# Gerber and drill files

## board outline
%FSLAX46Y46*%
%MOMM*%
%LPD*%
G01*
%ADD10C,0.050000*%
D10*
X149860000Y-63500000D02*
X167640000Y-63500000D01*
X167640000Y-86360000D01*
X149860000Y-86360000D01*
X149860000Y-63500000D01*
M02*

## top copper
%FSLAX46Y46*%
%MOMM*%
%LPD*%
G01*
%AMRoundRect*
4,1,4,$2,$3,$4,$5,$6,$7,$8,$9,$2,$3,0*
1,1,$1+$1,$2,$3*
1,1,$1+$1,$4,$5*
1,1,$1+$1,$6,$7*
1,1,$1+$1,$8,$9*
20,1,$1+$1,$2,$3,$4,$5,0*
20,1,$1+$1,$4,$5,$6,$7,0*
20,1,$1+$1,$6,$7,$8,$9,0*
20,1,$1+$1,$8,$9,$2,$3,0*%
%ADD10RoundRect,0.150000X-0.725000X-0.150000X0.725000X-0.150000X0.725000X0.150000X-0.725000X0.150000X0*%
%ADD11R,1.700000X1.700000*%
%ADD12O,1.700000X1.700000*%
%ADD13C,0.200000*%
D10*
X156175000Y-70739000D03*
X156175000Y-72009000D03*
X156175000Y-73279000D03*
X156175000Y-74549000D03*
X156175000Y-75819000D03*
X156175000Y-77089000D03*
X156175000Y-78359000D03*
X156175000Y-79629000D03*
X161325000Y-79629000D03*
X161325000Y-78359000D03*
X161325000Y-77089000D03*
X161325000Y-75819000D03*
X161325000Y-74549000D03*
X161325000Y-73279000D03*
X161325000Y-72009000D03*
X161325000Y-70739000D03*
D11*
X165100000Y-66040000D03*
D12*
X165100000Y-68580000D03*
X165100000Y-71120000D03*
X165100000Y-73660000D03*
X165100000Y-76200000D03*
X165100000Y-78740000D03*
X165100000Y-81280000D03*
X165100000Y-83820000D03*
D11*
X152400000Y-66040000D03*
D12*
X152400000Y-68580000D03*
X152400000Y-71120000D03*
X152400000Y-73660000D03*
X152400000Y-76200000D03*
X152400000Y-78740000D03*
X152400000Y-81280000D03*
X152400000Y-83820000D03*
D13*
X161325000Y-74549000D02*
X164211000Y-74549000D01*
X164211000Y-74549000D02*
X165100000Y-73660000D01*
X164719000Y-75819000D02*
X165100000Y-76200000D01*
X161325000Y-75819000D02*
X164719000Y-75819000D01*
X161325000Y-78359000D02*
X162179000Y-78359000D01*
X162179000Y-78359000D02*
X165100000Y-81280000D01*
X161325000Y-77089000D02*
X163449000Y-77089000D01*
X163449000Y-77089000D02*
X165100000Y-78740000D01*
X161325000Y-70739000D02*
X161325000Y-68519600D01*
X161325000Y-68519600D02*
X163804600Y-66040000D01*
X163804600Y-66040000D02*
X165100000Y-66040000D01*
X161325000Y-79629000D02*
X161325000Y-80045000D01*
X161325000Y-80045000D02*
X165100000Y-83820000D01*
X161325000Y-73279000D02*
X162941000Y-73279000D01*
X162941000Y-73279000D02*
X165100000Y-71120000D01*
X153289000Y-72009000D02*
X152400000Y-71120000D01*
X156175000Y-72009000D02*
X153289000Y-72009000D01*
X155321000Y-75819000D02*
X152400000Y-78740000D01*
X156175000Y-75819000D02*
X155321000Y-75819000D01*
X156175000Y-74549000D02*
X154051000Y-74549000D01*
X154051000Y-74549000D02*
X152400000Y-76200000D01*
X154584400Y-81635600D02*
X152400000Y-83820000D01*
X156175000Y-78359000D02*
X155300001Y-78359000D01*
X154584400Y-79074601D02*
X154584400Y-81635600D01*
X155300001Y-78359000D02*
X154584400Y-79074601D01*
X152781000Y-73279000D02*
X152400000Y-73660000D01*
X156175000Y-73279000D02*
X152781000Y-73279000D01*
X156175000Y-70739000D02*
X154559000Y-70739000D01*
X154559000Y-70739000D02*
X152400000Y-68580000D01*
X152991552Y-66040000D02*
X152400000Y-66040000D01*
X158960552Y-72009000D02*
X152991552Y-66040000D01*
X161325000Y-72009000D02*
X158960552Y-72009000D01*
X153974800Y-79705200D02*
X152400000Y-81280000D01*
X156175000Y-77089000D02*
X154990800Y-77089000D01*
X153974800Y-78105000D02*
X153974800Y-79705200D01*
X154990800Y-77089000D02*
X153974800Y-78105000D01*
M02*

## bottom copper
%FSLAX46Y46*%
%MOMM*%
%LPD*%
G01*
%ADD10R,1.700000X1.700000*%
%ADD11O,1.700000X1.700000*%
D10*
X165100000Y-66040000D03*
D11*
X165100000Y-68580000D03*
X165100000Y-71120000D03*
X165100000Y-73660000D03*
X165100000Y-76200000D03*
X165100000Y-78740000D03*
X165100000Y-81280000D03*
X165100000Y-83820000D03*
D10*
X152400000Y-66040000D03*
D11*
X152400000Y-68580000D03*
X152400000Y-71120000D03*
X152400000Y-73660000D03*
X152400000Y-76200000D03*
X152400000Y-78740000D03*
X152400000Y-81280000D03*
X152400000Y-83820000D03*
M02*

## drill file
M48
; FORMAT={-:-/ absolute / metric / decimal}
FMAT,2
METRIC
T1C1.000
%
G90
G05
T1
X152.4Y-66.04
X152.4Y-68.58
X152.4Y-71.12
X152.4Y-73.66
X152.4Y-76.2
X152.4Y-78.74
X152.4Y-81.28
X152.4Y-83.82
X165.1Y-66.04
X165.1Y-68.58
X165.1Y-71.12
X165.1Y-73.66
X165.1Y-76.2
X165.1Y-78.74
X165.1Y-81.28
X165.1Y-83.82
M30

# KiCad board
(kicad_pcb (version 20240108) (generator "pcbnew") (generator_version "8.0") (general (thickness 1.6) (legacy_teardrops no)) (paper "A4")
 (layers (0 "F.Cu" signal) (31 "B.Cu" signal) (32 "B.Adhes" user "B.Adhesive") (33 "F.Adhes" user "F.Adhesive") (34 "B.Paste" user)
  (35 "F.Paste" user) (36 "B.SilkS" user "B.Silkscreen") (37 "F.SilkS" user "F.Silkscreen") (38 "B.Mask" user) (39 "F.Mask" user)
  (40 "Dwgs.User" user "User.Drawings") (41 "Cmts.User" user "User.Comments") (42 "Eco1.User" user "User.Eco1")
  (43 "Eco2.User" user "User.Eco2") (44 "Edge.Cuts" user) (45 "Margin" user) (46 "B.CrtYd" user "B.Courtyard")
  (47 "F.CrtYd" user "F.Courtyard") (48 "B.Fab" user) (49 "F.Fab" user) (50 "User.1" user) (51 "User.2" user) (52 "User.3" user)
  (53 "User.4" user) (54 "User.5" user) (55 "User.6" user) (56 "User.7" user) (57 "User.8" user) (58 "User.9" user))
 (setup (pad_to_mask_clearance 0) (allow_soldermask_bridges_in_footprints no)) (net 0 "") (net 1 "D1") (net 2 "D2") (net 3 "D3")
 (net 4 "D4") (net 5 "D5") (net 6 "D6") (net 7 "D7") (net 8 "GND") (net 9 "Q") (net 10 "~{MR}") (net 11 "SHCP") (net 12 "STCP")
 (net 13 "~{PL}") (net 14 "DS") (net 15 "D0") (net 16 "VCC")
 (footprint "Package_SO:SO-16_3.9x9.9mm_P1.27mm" (layer "F.Cu") (at 158.75 75.184)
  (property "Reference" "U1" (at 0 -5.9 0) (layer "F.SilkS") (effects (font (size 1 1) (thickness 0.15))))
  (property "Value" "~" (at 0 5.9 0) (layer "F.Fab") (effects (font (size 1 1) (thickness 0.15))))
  (pad "1" smd roundrect (at -2.575 -4.445) (size 1.75 0.6) (layers "F.Cu" "F.Paste" "F.Mask") (roundrect_rratio 0.25) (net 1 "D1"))
  (pad "2" smd roundrect (at -2.575 -3.175) (size 1.75 0.6) (layers "F.Cu" "F.Paste" "F.Mask") (roundrect_rratio 0.25) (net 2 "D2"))
  (pad "3" smd roundrect (at -2.575 -1.905) (size 1.75 0.6) (layers "F.Cu" "F.Paste" "F.Mask") (roundrect_rratio 0.25) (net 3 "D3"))
  (pad "4" smd roundrect (at -2.575 -0.635) (size 1.75 0.6) (layers "F.Cu" "F.Paste" "F.Mask") (roundrect_rratio 0.25) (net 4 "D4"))
  (pad "5" smd roundrect (at -2.575 0.635) (size 1.75 0.6) (layers "F.Cu" "F.Paste" "F.Mask") (roundrect_rratio 0.25) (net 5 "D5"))
  (pad "6" smd roundrect (at -2.575 1.905) (size 1.75 0.6) (layers "F.Cu" "F.Paste" "F.Mask") (roundrect_rratio 0.25) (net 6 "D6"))
  (pad "7" smd roundrect (at -2.575 3.175) (size 1.75 0.6) (layers "F.Cu" "F.Paste" "F.Mask") (roundrect_rratio 0.25) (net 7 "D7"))
  (pad "8" smd roundrect (at -2.575 4.445) (size 1.75 0.6) (layers "F.Cu" "F.Paste" "F.Mask") (roundrect_rratio 0.25) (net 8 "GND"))
  (pad "9" smd roundrect (at 2.575 4.445) (size 1.75 0.6) (layers "F.Cu" "F.Paste" "F.Mask") (roundrect_rratio 0.25) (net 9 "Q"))
  (pad "10" smd roundrect (at 2.575 3.175) (size 1.75 0.6) (layers "F.Cu" "F.Paste" "F.Mask") (roundrect_rratio 0.25) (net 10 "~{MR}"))
  (pad "11" smd roundrect (at 2.575 1.905) (size 1.75 0.6) (layers "F.Cu" "F.Paste" "F.Mask") (roundrect_rratio 0.25) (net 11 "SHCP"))
  (pad "12" smd roundrect (at 2.575 0.635) (size 1.75 0.6) (layers "F.Cu" "F.Paste" "F.Mask") (roundrect_rratio 0.25) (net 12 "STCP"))
  (pad "13" smd roundrect (at 2.575 -0.635) (size 1.75 0.6) (layers "F.Cu" "F.Paste" "F.Mask") (roundrect_rratio 0.25) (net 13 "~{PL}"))
  (pad "14" smd roundrect (at 2.575 -1.905) (size 1.75 0.6) (layers "F.Cu" "F.Paste" "F.Mask") (roundrect_rratio 0.25) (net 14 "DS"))
  (pad "15" smd roundrect (at 2.575 -3.175) (size 1.75 0.6) (layers "F.Cu" "F.Paste" "F.Mask") (roundrect_rratio 0.25) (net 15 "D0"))
  (pad "16" smd roundrect (at 2.575 -4.445) (size 1.75 0.6) (layers "F.Cu" "F.Paste" "F.Mask") (roundrect_rratio 0.25) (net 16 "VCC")))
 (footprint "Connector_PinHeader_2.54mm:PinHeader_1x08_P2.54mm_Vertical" (layer "B.Cu") (at 165.1 66.04 180)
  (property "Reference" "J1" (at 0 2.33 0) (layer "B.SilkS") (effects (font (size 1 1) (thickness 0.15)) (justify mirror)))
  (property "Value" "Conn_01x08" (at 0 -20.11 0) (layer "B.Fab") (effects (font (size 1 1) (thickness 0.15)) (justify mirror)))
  (pad "1" thru_hole rect (at 0 0 180) (size 1.7 1.7) (drill 1) (layers "*.Cu" "*.Mask") (remove_unused_layers no) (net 16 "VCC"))
  (pad "2" thru_hole oval (at 0 -2.54 180) (size 1.7 1.7) (drill 1) (layers "*.Cu" "*.Mask") (remove_unused_layers no) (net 8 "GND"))
  (pad "3" thru_hole oval (at 0 -5.08 180) (size 1.7 1.7) (drill 1) (layers "*.Cu" "*.Mask") (remove_unused_layers no) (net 14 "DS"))
  (pad "4" thru_hole oval (at 0 -7.62 180) (size 1.7 1.7) (drill 1) (layers "*.Cu" "*.Mask") (remove_unused_layers no) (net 13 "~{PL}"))
  (pad "5" thru_hole oval (at 0 -10.16 180) (size 1.7 1.7) (drill 1) (layers "*.Cu" "*.Mask") (remove_unused_layers no) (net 12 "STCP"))
  (pad "6" thru_hole oval (at 0 -12.7 180) (size 1.7 1.7) (drill 1) (layers "*.Cu" "*.Mask") (remove_unused_layers no) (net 11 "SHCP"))
  (pad "7" thru_hole oval (at 0 -15.24 180) (size 1.7 1.7) (drill 1) (layers "*.Cu" "*.Mask") (remove_unused_layers no) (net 10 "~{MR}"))
  (pad "8" thru_hole oval (at 0 -17.78 180) (size 1.7 1.7) (drill 1) (layers "*.Cu" "*.Mask") (remove_unused_layers no) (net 9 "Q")))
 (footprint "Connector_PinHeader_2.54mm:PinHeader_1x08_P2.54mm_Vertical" (layer "B.Cu") (at 152.4 66.04 180)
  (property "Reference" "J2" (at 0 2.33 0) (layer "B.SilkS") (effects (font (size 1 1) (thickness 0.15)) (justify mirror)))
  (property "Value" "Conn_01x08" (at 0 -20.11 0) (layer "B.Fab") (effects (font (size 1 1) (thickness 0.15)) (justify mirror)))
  (pad "1" thru_hole rect (at 0 0 180) (size 1.7 1.7) (drill 1) (layers "*.Cu" "*.Mask") (remove_unused_layers no) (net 15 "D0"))
  (pad "2" thru_hole oval (at 0 -2.54 180) (size 1.7 1.7) (drill 1) (layers "*.Cu" "*.Mask") (remove_unused_layers no) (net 1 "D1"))
  (pad "3" thru_hole oval (at 0 -5.08 180) (size 1.7 1.7) (drill 1) (layers "*.Cu" "*.Mask") (remove_unused_layers no) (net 2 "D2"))
  (pad "4" thru_hole oval (at 0 -7.62 180) (size 1.7 1.7) (drill 1) (layers "*.Cu" "*.Mask") (remove_unused_layers no) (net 3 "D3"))
  (pad "5" thru_hole oval (at 0 -10.16 180) (size 1.7 1.7) (drill 1) (layers "*.Cu" "*.Mask") (remove_unused_layers no) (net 4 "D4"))
  (pad "6" thru_hole oval (at 0 -12.7 180) (size 1.7 1.7) (drill 1) (layers "*.Cu" "*.Mask") (remove_unused_layers no) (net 5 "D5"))
  (pad "7" thru_hole oval (at 0 -15.24 180) (size 1.7 1.7) (drill 1) (layers "*.Cu" "*.Mask") (remove_unused_layers no) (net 6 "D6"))
  (pad "8" thru_hole oval (at 0 -17.78 180) (size 1.7 1.7) (drill 1) (layers "*.Cu" "*.Mask") (remove_unused_layers no) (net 7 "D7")))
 (gr_rect (start 149.86 63.5) (end 167.64 86.36) (stroke (width 0.05) (type default)) (fill none) (layer "Edge.Cuts"))
 (segment (start 161.325 74.549) (end 164.211 74.549) (width 0.2) (layer "F.Cu") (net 13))
 (segment (start 164.211 74.549) (end 165.1 73.66) (width 0.2) (layer "F.Cu") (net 13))
 (segment (start 164.719 75.819) (end 165.1 76.2) (width 0.2) (layer "F.Cu") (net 12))
 (segment (start 161.325 75.819) (end 164.719 75.819) (width 0.2) (layer "F.Cu") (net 12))
 (segment (start 161.325 78.359) (end 162.179 78.359) (width 0.2) (layer "F.Cu") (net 10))
 (segment (start 162.179 78.359) (end 165.1 81.28) (width 0.2) (layer "F.Cu") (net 10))
 (segment (start 161.325 77.089) (end 163.449 77.089) (width 0.2) (layer "F.Cu") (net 11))
 (segment (start 163.449 77.089) (end 165.1 78.74) (width 0.2) (layer "F.Cu") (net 11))
 (segment (start 161.325 70.739) (end 161.325 68.5196) (width 0.2) (layer "F.Cu") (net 16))
 (segment (start 161.325 68.5196) (end 163.8046 66.04) (width 0.2) (layer "F.Cu") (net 16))
 (segment (start 163.8046 66.04) (end 165.1 66.04) (width 0.2) (layer "F.Cu") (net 16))
 (segment (start 161.325 79.629) (end 161.325 80.045) (width 0.2) (layer "F.Cu") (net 9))
 (segment (start 161.325 80.045) (end 165.1 83.82) (width 0.2) (layer "F.Cu") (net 9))
 (segment (start 161.325 73.279) (end 162.941 73.279) (width 0.2) (layer "F.Cu") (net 14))
 (segment (start 162.941 73.279) (end 165.1 71.12) (width 0.2) (layer "F.Cu") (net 14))
 (segment (start 153.289 72.009) (end 152.4 71.12) (width 0.2) (layer "F.Cu") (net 2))
 (segment (start 156.175 72.009) (end 153.289 72.009) (width 0.2) (layer "F.Cu") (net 2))
 (segment (start 155.321 75.819) (end 152.4 78.74) (width 0.2) (layer "F.Cu") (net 5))
 (segment (start 156.175 75.819) (end 155.321 75.819) (width 0.2) (layer "F.Cu") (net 5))
 (segment (start 156.175 74.549) (end 154.051 74.549) (width 0.2) (layer "F.Cu") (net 4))
 (segment (start 154.051 74.549) (end 152.4 76.2) (width 0.2) (layer "F.Cu") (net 4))
 (segment (start 154.5844 81.6356) (end 152.4 83.82) (width 0.2) (layer "F.Cu") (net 7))
 (segment (start 156.175 78.359) (end 155.300001 78.359) (width 0.2) (layer "F.Cu") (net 7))
 (segment (start 154.5844 79.074601) (end 154.5844 81.6356) (width 0.2) (layer "F.Cu") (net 7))
 (segment (start 155.300001 78.359) (end 154.5844 79.074601) (width 0.2) (layer "F.Cu") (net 7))
 (segment (start 152.781 73.279) (end 152.4 73.66) (width 0.2) (layer "F.Cu") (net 3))
 (segment (start 156.175 73.279) (end 152.781 73.279) (width 0.2) (layer "F.Cu") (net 3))
 (segment (start 156.175 70.739) (end 154.559 70.739) (width 0.2) (layer "F.Cu") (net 1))
 (segment (start 154.559 70.739) (end 152.4 68.58) (width 0.2) (layer "F.Cu") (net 1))
 (segment (start 152.991552 66.04) (end 152.4 66.04) (width 0.2) (layer "F.Cu") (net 15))
 (segment (start 158.960552 72.009) (end 152.991552 66.04) (width 0.2) (layer "F.Cu") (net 15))
 (segment (start 161.325 72.009) (end 158.960552 72.009) (width 0.2) (layer "F.Cu") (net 15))
 (segment (start 153.9748 79.7052) (end 152.4 81.28) (width 0.2) (layer "F.Cu") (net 6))
 (segment (start 156.175 77.089) (end 154.9908 77.089) (width 0.2) (layer "F.Cu") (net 6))
 (segment (start 153.9748 78.105) (end 153.9748 79.7052) (width 0.2) (layer "F.Cu") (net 6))
 (segment (start 154.9908 77.089) (end 153.9748 78.105) (width 0.2) (layer "F.Cu") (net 6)))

